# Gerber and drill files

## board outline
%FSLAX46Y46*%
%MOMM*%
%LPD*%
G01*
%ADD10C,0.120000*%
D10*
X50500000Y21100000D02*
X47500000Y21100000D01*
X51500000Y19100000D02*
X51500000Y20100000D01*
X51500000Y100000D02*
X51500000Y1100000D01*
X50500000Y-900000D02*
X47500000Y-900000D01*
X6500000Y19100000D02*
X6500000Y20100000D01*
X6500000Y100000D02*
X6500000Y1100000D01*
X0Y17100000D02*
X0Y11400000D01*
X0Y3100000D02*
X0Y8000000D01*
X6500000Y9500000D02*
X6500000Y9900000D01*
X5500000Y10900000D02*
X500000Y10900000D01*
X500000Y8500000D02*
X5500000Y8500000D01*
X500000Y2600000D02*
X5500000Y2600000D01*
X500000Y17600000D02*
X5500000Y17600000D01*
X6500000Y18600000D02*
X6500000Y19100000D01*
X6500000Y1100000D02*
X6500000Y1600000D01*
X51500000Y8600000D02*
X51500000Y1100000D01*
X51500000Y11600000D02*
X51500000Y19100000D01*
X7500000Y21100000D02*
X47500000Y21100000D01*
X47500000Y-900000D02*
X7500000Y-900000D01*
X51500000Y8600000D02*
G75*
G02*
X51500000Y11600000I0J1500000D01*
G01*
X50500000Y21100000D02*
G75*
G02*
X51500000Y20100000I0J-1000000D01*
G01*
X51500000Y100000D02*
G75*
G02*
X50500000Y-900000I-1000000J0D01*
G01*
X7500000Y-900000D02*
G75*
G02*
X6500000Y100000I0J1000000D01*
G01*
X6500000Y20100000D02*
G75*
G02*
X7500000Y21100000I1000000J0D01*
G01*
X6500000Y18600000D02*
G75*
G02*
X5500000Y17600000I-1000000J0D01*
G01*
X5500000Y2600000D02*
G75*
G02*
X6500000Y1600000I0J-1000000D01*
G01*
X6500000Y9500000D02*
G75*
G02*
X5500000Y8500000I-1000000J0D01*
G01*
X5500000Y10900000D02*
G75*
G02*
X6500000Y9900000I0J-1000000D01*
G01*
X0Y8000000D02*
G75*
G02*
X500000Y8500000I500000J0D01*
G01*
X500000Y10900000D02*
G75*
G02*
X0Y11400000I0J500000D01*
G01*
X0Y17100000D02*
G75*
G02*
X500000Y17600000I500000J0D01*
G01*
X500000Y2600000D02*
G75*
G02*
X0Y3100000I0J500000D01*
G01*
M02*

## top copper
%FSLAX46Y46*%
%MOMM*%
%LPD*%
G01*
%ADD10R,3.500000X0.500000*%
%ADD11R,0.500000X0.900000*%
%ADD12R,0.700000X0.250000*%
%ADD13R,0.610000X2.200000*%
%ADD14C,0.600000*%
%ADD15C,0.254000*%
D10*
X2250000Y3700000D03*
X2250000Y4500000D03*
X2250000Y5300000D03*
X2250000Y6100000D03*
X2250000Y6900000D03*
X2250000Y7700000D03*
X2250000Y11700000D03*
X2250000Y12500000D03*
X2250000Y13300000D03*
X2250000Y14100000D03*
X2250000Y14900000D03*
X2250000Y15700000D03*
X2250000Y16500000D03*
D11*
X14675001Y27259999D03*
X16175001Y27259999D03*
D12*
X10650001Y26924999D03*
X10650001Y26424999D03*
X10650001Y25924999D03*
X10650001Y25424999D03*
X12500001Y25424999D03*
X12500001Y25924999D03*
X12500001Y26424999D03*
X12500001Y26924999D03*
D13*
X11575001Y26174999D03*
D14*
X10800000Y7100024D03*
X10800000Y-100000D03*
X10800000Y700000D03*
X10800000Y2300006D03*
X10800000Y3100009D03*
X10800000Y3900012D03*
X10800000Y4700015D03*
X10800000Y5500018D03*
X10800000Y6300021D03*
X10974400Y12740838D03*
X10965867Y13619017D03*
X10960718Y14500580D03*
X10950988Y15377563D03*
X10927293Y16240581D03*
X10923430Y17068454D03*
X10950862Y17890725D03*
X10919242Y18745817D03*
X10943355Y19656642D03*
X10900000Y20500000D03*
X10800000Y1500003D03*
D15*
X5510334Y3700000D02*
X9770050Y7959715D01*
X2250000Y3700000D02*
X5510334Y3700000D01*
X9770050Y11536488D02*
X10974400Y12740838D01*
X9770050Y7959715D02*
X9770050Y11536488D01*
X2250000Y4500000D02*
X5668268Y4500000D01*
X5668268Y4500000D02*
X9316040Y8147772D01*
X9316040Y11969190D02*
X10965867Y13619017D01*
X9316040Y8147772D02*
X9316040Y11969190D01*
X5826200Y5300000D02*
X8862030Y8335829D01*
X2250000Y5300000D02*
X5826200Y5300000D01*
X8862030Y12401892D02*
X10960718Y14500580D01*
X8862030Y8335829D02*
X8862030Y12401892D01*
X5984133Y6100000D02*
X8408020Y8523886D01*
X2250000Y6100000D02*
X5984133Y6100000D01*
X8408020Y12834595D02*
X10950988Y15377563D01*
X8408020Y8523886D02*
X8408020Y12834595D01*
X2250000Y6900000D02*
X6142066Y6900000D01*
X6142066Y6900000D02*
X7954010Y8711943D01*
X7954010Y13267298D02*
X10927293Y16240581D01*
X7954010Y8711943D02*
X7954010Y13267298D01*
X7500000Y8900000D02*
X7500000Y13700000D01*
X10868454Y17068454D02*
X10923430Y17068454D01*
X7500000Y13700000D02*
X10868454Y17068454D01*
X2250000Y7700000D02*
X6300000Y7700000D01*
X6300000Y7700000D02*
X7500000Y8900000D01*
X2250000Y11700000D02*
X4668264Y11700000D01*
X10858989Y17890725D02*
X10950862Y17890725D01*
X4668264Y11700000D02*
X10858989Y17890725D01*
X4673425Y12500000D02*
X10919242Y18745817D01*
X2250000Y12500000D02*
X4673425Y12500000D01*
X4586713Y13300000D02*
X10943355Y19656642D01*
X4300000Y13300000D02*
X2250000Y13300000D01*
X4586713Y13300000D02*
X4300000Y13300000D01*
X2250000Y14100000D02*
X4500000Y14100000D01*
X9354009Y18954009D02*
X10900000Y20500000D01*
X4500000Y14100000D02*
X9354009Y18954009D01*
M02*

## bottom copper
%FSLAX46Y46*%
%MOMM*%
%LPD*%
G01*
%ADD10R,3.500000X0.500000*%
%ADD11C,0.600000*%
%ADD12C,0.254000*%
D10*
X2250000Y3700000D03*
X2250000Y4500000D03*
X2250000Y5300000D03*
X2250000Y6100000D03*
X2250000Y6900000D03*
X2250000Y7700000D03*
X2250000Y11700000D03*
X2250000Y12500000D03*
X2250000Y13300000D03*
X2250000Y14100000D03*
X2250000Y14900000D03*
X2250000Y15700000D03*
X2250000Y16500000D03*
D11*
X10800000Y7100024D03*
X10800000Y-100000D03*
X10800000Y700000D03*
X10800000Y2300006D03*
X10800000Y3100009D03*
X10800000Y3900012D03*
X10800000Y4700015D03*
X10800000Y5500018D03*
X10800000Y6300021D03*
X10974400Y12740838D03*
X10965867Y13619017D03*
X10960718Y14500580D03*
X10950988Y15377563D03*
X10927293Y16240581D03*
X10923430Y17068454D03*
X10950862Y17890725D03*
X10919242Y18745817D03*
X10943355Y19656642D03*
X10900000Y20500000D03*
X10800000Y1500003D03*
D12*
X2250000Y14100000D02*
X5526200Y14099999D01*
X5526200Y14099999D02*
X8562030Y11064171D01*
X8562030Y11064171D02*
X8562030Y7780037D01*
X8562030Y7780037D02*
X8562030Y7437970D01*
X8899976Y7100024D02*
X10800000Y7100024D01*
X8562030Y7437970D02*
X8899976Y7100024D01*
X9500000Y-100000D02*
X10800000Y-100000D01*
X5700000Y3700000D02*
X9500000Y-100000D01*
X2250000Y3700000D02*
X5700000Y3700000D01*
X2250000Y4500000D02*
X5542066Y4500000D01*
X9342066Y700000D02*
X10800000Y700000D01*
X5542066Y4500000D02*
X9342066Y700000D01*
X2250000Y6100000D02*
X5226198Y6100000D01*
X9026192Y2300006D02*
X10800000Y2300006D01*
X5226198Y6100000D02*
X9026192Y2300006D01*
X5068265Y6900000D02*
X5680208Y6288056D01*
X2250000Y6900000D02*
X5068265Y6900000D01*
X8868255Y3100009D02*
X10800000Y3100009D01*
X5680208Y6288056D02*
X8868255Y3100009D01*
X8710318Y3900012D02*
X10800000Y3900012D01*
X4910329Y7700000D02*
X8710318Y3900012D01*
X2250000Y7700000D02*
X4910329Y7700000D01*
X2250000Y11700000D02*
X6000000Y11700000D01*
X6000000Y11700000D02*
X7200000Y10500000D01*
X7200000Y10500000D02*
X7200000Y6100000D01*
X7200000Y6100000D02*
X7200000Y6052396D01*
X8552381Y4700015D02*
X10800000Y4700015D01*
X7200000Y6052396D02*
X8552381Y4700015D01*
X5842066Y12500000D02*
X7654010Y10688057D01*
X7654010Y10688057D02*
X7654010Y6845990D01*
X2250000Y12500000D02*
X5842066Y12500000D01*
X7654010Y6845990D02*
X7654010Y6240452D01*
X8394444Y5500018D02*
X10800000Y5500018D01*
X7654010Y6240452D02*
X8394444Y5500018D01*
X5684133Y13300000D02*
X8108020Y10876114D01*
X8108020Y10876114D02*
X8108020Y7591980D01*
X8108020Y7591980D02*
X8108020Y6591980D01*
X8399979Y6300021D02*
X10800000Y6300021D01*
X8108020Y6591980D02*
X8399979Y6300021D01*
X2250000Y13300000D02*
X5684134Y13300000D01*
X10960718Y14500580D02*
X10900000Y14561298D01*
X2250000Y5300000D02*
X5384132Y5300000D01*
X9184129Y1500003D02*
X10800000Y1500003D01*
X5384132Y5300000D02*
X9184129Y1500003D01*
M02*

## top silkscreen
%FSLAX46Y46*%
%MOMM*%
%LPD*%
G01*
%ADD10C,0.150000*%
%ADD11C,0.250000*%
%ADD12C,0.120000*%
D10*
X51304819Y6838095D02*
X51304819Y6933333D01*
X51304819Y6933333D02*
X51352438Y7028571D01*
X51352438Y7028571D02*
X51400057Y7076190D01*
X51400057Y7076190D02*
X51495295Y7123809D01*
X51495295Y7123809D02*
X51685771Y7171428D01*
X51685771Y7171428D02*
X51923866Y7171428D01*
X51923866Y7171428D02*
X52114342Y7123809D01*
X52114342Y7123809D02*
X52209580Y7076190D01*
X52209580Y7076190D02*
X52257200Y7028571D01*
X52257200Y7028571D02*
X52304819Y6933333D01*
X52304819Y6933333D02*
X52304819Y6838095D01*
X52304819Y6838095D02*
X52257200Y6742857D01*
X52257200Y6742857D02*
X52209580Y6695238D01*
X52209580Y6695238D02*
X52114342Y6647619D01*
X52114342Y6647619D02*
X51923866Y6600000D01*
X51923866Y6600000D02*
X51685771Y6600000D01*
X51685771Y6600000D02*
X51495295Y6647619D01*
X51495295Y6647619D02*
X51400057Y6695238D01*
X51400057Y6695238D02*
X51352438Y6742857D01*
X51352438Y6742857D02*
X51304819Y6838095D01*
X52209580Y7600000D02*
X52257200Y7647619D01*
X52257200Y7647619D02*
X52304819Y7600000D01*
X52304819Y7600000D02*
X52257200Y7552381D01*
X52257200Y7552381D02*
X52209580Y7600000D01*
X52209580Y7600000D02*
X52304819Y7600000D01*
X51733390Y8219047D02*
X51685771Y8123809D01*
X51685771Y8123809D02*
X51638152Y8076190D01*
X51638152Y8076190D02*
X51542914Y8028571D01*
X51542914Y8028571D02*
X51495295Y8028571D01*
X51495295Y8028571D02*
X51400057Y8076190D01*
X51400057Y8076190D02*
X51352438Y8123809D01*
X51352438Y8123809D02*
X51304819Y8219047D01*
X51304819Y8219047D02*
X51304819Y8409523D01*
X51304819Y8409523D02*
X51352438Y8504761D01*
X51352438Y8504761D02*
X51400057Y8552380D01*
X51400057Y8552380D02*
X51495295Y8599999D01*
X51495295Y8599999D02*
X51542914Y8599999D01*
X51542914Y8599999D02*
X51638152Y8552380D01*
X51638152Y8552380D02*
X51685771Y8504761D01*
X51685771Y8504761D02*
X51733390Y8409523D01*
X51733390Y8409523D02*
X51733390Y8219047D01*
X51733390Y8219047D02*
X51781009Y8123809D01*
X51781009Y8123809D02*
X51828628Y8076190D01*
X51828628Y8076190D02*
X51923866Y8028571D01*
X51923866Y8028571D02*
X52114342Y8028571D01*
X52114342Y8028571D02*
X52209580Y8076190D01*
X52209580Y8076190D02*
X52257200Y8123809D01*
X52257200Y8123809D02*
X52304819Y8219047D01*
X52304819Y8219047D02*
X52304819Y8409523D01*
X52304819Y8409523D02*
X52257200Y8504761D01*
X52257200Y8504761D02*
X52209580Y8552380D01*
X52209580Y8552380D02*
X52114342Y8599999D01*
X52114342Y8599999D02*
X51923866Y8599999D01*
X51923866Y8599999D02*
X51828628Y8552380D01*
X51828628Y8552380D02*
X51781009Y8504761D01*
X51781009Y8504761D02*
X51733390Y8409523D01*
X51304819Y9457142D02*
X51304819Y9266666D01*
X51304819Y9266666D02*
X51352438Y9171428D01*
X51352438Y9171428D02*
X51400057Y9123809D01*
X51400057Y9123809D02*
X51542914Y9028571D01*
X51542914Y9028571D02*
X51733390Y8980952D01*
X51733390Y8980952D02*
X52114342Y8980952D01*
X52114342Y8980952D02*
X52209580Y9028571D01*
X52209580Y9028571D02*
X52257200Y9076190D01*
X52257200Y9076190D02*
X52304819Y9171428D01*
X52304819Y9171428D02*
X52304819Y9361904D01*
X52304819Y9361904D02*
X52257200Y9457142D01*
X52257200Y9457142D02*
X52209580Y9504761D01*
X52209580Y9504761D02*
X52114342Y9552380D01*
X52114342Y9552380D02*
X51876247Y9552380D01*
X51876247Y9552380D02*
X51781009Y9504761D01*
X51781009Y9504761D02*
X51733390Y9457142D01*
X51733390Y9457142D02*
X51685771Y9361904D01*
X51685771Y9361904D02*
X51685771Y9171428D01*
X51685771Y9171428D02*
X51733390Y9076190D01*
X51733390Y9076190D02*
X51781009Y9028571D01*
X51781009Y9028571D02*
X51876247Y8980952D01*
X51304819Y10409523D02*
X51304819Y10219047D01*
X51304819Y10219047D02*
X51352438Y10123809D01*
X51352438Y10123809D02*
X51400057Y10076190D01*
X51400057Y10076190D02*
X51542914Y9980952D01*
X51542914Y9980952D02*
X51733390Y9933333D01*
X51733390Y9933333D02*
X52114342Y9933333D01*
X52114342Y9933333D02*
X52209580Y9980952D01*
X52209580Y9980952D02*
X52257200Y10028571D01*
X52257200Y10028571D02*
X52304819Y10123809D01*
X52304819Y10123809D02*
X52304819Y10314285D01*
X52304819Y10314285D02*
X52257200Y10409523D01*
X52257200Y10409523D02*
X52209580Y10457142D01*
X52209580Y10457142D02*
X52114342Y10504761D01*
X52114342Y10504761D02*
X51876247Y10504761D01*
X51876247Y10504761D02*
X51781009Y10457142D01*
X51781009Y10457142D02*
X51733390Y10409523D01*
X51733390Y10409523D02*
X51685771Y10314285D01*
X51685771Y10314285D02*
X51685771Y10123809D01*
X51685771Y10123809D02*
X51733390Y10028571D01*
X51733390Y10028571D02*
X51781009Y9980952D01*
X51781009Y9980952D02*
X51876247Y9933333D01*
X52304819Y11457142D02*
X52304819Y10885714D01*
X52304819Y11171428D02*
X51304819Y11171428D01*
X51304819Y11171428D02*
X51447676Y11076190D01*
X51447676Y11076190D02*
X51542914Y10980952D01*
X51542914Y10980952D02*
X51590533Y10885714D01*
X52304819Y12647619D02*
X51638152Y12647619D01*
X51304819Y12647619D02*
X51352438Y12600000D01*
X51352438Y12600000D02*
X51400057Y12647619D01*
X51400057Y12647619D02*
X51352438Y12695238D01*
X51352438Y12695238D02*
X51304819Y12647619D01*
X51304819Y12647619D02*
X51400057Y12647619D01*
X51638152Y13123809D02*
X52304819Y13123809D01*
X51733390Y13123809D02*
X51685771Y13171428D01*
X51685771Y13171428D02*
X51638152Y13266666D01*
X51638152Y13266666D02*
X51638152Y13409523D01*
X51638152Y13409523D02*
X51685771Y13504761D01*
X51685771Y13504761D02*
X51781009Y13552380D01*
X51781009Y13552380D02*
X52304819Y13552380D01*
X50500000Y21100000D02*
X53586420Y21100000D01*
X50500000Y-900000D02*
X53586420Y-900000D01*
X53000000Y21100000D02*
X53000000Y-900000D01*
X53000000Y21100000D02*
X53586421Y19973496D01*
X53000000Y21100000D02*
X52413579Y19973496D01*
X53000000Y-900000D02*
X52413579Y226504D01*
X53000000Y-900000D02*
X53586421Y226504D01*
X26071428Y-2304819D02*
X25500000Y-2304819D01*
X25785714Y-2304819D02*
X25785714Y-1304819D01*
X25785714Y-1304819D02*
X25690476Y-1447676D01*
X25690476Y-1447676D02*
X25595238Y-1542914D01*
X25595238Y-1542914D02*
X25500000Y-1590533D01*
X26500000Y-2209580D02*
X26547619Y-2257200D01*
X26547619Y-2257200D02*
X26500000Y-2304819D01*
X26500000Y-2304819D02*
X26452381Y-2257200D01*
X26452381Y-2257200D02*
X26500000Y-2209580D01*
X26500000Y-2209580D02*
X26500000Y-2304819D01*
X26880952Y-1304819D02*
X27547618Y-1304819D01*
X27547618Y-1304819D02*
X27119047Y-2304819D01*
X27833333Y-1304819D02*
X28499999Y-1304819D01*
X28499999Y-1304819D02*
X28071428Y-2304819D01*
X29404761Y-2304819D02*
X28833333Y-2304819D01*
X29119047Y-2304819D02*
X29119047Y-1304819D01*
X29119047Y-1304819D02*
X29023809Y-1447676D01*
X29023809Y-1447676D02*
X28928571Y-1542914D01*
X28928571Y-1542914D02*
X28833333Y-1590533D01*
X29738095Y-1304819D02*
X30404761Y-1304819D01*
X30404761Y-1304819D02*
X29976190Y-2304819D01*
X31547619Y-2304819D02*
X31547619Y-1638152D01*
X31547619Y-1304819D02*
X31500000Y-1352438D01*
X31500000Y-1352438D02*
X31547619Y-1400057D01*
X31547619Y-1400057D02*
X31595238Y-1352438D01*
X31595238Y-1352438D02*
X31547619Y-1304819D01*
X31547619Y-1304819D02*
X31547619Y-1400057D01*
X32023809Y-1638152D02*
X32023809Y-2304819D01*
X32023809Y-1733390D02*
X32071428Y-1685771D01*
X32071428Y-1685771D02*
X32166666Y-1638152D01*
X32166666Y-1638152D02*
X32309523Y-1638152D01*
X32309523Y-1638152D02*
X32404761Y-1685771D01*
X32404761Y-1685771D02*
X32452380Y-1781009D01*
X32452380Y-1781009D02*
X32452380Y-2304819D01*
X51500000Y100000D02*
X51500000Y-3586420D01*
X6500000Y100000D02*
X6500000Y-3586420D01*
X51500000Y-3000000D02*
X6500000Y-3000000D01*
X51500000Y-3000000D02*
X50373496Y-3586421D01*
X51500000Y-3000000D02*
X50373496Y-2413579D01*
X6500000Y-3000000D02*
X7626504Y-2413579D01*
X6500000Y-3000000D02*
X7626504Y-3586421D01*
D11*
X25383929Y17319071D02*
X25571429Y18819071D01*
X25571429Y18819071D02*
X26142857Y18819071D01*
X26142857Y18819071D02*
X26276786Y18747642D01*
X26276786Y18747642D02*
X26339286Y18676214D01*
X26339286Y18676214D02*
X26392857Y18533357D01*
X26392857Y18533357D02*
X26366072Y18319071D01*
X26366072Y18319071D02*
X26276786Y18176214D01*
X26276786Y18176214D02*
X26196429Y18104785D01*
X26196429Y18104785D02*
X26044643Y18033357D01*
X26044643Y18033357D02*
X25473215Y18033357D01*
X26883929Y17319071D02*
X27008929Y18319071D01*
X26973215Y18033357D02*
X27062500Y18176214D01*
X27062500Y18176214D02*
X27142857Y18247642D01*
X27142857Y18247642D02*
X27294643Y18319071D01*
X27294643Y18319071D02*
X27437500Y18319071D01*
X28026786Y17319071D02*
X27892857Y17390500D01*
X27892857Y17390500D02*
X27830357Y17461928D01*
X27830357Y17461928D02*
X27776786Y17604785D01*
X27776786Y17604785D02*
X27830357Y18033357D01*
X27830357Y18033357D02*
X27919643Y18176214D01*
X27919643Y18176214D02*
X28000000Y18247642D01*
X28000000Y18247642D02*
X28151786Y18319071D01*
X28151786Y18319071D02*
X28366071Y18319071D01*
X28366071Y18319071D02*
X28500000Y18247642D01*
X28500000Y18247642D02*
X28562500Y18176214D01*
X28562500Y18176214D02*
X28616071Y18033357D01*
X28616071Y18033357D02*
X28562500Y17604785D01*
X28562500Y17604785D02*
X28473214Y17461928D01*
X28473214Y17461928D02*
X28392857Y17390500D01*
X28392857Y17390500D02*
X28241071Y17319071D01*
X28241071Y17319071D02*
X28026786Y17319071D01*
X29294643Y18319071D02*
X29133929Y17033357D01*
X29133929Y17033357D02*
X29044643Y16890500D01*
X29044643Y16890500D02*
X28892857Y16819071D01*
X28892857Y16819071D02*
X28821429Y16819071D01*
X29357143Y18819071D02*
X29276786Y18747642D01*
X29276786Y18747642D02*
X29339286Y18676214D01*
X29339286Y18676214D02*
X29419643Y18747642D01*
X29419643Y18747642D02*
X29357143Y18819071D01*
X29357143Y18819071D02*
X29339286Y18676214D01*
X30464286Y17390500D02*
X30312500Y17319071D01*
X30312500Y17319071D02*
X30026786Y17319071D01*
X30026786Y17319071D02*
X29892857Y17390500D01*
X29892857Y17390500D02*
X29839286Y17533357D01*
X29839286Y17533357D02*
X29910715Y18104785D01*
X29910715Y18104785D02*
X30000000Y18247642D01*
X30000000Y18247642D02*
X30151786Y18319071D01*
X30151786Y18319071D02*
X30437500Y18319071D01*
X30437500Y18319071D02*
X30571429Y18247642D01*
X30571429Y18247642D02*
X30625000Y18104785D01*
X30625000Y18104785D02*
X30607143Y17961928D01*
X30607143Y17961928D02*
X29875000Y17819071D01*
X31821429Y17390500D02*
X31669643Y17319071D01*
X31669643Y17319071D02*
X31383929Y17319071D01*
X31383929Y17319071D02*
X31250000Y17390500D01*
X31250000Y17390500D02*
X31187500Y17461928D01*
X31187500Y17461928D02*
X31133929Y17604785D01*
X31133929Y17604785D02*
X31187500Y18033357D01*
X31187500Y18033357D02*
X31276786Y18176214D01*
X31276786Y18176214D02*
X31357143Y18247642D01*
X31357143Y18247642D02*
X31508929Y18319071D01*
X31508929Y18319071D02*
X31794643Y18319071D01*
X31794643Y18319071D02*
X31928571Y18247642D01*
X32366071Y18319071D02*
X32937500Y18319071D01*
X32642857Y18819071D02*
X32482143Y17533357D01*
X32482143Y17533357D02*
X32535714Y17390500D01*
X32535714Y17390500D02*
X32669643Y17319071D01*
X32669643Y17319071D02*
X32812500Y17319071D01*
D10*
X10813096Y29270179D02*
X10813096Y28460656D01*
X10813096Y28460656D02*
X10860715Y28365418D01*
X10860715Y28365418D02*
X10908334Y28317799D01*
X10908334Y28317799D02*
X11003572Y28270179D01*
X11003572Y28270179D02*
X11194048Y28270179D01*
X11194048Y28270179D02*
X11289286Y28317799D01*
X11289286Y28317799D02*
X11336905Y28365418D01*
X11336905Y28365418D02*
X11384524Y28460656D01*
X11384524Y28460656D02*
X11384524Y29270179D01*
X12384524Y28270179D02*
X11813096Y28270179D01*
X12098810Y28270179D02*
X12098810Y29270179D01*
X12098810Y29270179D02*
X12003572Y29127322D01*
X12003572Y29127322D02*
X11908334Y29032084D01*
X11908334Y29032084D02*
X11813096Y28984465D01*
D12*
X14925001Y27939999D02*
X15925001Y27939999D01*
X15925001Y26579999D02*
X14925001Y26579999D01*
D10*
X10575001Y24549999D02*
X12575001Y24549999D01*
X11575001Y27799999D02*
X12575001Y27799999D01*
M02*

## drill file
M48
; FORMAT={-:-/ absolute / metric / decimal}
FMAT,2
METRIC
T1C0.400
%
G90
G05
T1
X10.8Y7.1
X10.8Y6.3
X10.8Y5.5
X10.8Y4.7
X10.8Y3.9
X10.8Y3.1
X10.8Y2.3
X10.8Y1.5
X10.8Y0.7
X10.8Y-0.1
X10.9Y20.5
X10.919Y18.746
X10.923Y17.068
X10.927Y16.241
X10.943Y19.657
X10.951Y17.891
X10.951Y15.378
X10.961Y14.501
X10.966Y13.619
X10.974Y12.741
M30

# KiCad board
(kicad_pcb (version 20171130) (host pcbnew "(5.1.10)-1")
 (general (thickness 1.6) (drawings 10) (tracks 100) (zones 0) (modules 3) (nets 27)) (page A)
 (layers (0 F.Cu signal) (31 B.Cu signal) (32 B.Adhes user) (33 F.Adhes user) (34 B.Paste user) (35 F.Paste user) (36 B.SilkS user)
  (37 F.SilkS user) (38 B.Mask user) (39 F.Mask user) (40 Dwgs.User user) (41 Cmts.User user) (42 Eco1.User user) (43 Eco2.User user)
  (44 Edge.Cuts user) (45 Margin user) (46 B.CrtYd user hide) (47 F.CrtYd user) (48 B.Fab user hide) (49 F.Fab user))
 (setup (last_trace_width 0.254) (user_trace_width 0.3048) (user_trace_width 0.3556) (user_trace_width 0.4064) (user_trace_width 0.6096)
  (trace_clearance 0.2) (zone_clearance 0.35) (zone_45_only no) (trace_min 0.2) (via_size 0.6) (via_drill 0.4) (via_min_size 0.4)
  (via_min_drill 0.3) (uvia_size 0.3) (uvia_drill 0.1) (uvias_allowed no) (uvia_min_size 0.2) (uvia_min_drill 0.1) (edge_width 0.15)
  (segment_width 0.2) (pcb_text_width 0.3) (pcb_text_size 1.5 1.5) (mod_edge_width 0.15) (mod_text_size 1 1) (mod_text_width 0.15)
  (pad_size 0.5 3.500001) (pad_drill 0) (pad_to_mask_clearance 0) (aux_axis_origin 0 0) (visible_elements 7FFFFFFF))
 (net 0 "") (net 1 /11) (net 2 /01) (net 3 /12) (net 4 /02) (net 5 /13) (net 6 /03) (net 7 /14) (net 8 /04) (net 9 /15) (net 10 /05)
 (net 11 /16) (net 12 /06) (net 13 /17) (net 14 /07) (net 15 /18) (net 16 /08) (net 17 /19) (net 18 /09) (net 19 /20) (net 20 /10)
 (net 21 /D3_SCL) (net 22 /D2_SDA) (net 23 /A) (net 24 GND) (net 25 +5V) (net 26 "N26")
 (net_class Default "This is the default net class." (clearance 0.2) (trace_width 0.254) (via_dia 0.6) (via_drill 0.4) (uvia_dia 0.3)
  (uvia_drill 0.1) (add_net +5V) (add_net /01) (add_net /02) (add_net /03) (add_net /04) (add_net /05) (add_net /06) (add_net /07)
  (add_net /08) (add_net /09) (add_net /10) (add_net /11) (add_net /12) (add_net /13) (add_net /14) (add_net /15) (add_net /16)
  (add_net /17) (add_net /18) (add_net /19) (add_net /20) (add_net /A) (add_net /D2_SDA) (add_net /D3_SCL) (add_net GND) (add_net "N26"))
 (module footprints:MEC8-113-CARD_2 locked (layer F.Cu) (at 0 -0.1 90)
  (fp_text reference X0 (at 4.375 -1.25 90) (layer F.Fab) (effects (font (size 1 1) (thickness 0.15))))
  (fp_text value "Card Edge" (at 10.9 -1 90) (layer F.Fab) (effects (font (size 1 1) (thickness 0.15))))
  (fp_line (start 21 50.5) (end 21 47.5) (layer Edge.Cuts) (width 0.12))
  (fp_line (start 19 51.5) (end 20 51.5) (layer Edge.Cuts) (width 0.12))
  (fp_line (start 0 51.5) (end 1 51.5) (layer Edge.Cuts) (width 0.12))
  (fp_line (start -1 50.5) (end -1 47.5) (layer Edge.Cuts) (width 0.12))
  (fp_line (start 19 6.5) (end 20 6.5) (layer Edge.Cuts) (width 0.12))
  (fp_line (start 0 6.5) (end 1 6.5) (layer Edge.Cuts) (width 0.12))
  (fp_line (start 17 0) (end 11.3 0) (layer Edge.Cuts) (width 0.12))
  (fp_line (start 3 0) (end 7.9 0) (layer Edge.Cuts) (width 0.12))
  (fp_line (start 9.4 6.5) (end 9.8 6.5) (layer Edge.Cuts) (width 0.12))
  (fp_line (start 10.8 5.5) (end 10.8 0.5) (layer Edge.Cuts) (width 0.12))
  (fp_line (start 8.4 0.5) (end 8.4 5.5) (layer Edge.Cuts) (width 0.12))
  (fp_line (start 2.5 0.5) (end 2.5 5.5) (layer Edge.Cuts) (width 0.12))
  (fp_line (start 17.5 0.5) (end 17.5 5.5) (layer Edge.Cuts) (width 0.12))
  (fp_line (start 18.5 6.5) (end 19 6.5) (layer Edge.Cuts) (width 0.12))
  (fp_line (start 1 6.5) (end 1.5 6.5) (layer Edge.Cuts) (width 0.12))
  (fp_line (start 8.5 51.5) (end 1 51.5) (layer Edge.Cuts) (width 0.12))
  (fp_line (start 11.5 51.5) (end 19 51.5) (layer Edge.Cuts) (width 0.12))
  (fp_line (start 21 7.5) (end 21 47.5) (layer Edge.Cuts) (width 0.12))
  (fp_line (start -1 47.5) (end -1 7.5) (layer Edge.Cuts) (width 0.12))
  (fp_arc (start 10 51.5) (end 11.5 51.5) (angle -180) (layer Edge.Cuts) (width 0.12))
  (fp_arc (start 20 50.5) (end 20 51.5) (angle -90) (layer Edge.Cuts) (width 0.12))
  (fp_arc (start 0 50.5) (end -1 50.5) (angle -90) (layer Edge.Cuts) (width 0.12))
  (fp_arc (start 0 7.5) (end 0 6.5) (angle -90) (layer Edge.Cuts) (width 0.12))
  (fp_arc (start 20 7.5) (end 21 7.5) (angle -90) (layer Edge.Cuts) (width 0.12))
  (fp_arc (start 18.5 5.5) (end 17.5 5.5) (angle -90) (layer Edge.Cuts) (width 0.12))
  (fp_arc (start 1.5 5.5) (end 1.5 6.5) (angle -90) (layer Edge.Cuts) (width 0.12))
  (fp_arc (start 9.4 5.5) (end 8.4 5.5) (angle -90) (layer Edge.Cuts) (width 0.12))
  (fp_arc (start 9.8 5.5) (end 9.8 6.5) (angle -90) (layer Edge.Cuts) (width 0.12))
  (fp_arc (start 7.9 0.5) (end 8.4 0.5) (angle -90) (layer Edge.Cuts) (width 0.12))
  (fp_arc (start 11.3 0.5) (end 11.3 0) (angle -90) (layer Edge.Cuts) (width 0.12))
  (fp_arc (start 17 0.5) (end 17.5 0.5) (angle -90) (layer Edge.Cuts) (width 0.12))
  (fp_arc (start 3 0.5) (end 3 0) (angle -90) (layer Edge.Cuts) (width 0.12))
  (pad 14 smd rect (at 3.6 2.25 90) (size 0.5 3.5) (layers F.Cu F.Paste F.Mask) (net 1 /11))
  (pad 1 smd rect (at 3.6 2.25 90) (size 0.5 3.5) (layers B.Cu B.Paste B.Mask) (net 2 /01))
  (pad 15 smd rect (at 4.4 2.25 90) (size 0.5 3.5) (layers F.Cu F.Paste F.Mask) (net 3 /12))
  (pad 2 smd rect (at 4.4 2.25 90) (size 0.5 3.5) (layers B.Cu B.Paste B.Mask) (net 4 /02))
  (pad 16 smd rect (at 5.2 2.25 90) (size 0.5 3.5) (layers F.Cu F.Paste F.Mask) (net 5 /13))
  (pad 3 smd rect (at 5.2 2.25 90) (size 0.5 3.5) (layers B.Cu B.Paste B.Mask) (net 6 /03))
  (pad 17 smd rect (at 6 2.25 90) (size 0.5 3.5) (layers F.Cu F.Paste F.Mask) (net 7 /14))
  (pad 4 smd rect (at 6 2.25 90) (size 0.5 3.5) (layers B.Cu B.Paste B.Mask) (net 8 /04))
  (pad 18 smd rect (at 6.8 2.25 90) (size 0.5 3.5) (layers F.Cu F.Paste F.Mask) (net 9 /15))
  (pad 5 smd rect (at 6.8 2.25 90) (size 0.5 3.5) (layers B.Cu B.Paste B.Mask) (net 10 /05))
  (pad 19 smd rect (at 7.6 2.25 90) (size 0.5 3.5) (layers F.Cu F.Paste F.Mask) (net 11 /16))
  (pad 6 smd rect (at 7.6 2.25 90) (size 0.5 3.5) (layers B.Cu B.Paste B.Mask) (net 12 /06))
  (pad 20 smd rect (at 11.6 2.25 90) (size 0.5 3.5) (layers F.Cu F.Paste F.Mask) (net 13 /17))
  (pad 7 smd rect (at 11.6 2.25 90) (size 0.5 3.5) (layers B.Cu B.Paste B.Mask) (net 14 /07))
  (pad 21 smd rect (at 12.4 2.25 90) (size 0.5 3.5) (layers F.Cu F.Paste F.Mask) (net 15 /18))
  (pad 8 smd rect (at 12.4 2.25 90) (size 0.5 3.5) (layers B.Cu B.Paste B.Mask) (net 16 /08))
  (pad 22 smd rect (at 13.2 2.25 90) (size 0.5 3.5) (layers F.Cu F.Paste F.Mask) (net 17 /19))
  (pad 9 smd rect (at 13.2 2.25 90) (size 0.5 3.5) (layers B.Cu B.Paste B.Mask) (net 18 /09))
  (pad 23 smd rect (at 14 2.25 90) (size 0.5 3.5) (layers F.Cu F.Paste F.Mask) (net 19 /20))
  (pad 10 smd rect (at 14 2.25 90) (size 0.5 3.5) (layers B.Cu B.Paste B.Mask) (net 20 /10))
  (pad 24 smd rect (at 14.8 2.25 90) (size 0.5 3.5) (layers F.Cu F.Paste F.Mask) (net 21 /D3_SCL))
  (pad 11 smd rect (at 14.8 2.25 90) (size 0.5 3.5) (layers B.Cu B.Paste B.Mask))
  (pad 25 smd rect (at 15.6 2.25 90) (size 0.5 3.5) (layers F.Cu F.Paste F.Mask) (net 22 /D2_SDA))
  (pad 12 smd rect (at 15.6 2.25 90) (size 0.5 3.5) (layers B.Cu B.Paste B.Mask) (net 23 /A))
  (pad 26 smd rect (at 16.4 2.25 90) (size 0.5 3.5) (layers F.Cu F.Paste F.Mask) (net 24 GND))
  (pad 13 smd rect (at 16.4 2.25 90) (size 0.5 3.5) (layers B.Cu B.Paste B.Mask) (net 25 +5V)))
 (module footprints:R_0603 (layer F.Cu) (at 15.425001 -27.259999)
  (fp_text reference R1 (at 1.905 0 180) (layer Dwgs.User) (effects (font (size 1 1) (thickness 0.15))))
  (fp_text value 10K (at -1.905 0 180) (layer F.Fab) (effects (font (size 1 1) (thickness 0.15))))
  (fp_line (start -0.5 -0.68) (end 0.5 -0.68) (layer F.SilkS) (width 0.12))
  (fp_line (start 0.5 0.68) (end -0.5 0.68) (layer F.SilkS) (width 0.12))
  (pad 1 smd rect (at -0.75 0) (size 0.5 0.9) (layers F.Cu F.Paste F.Mask) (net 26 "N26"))
  (pad 2 smd rect (at 0.75 0) (size 0.5 0.9) (layers F.Cu F.Paste F.Mask) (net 23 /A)))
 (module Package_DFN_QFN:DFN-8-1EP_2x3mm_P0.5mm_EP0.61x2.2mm (layer F.Cu) (at 11.575001 -26.174999)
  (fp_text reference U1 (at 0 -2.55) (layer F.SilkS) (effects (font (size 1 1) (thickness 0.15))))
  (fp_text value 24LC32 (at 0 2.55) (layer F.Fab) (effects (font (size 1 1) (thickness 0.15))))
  (fp_line (start -1 1.625) (end 1 1.625) (layer F.SilkS) (width 0.15))
  (fp_line (start 0 -1.625) (end 1 -1.625) (layer F.SilkS) (width 0.15))
  (pad 1 smd rect (at -0.925 -0.75) (size 0.7 0.25) (layers F.Cu F.Paste F.Mask) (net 26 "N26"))
  (pad 2 smd rect (at -0.925 -0.25) (size 0.7 0.25) (layers F.Cu F.Paste F.Mask) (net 24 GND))
  (pad 3 smd rect (at -0.925 0.25) (size 0.7 0.25) (layers F.Cu F.Paste F.Mask) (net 24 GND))
  (pad 4 smd rect (at -0.925 0.75) (size 0.7 0.25) (layers F.Cu F.Paste F.Mask) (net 24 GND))
  (pad 5 smd rect (at 0.925 0.75) (size 0.7 0.25) (layers F.Cu F.Paste F.Mask) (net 22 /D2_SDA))
  (pad 6 smd rect (at 0.925 0.25) (size 0.7 0.25) (layers F.Cu F.Paste F.Mask) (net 21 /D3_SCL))
  (pad 7 smd rect (at 0.925 -0.25) (size 0.7 0.25) (layers F.Cu F.Paste F.Mask))
  (pad 8 smd rect (at 0.925 -0.75) (size 0.7 0.25) (layers F.Cu F.Paste F.Mask) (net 25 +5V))
  (pad 9 smd rect (at 0 0) (size 0.61 2.2) (layers F.Cu F.Mask))
  (pad "" smd rect (at 0 -0.734) (size 0.5 0.59) (layers F.Paste)) (pad "" smd rect (at 0 0) (size 0.5 0.59) (layers F.Paste))
  (pad "" smd rect (at 0 0.734) (size 0.5 0.59) (layers F.Paste)))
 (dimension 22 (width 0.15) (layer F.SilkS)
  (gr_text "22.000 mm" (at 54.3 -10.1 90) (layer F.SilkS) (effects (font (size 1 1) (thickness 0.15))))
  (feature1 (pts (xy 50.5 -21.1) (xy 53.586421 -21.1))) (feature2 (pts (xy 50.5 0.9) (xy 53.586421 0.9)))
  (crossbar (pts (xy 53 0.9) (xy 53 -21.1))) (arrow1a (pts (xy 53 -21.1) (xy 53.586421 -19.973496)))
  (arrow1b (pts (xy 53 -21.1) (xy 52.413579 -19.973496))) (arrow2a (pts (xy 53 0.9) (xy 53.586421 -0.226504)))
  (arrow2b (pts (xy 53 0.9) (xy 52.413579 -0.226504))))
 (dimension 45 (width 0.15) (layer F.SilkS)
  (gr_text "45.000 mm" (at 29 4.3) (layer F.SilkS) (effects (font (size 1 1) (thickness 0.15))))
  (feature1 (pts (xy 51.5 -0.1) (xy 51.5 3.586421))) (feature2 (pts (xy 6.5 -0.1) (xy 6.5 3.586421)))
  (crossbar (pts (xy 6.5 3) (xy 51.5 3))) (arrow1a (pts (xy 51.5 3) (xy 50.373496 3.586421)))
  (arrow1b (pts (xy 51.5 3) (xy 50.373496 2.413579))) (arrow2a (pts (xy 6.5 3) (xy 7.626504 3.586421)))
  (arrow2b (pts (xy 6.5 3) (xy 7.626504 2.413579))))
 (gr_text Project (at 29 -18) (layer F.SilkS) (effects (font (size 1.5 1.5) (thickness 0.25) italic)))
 (segment (start 2.25 -14.1) (end 5.5262 -14.099999) (width 0.254) (layer B.Cu) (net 20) (status 10))
 (segment (start 5.5262 -14.099999) (end 8.56203 -11.064171) (width 0.254) (layer B.Cu) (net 20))
 (segment (start 8.56203 -11.064171) (end 8.56203 -7.780037) (width 0.254) (layer B.Cu) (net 20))
 (segment (start 8.56203 -7.780037) (end 8.56203 -7.43797) (width 0.254) (layer B.Cu) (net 20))
 (via (at 10.8 -7.100024) (size 0.6) (drill 0.4) (layers F.Cu B.Cu) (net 20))
 (segment (start 8.899976 -7.100024) (end 10.8 -7.100024) (width 0.254) (layer B.Cu) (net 20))
 (segment (start 8.56203 -7.43797) (end 8.899976 -7.100024) (width 0.254) (layer B.Cu) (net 20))
 (via (at 10.8 0.1) (size 0.6) (drill 0.4) (layers F.Cu B.Cu) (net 2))
 (segment (start 9.5 0.1) (end 10.8 0.1) (width 0.254) (layer B.Cu) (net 2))
 (segment (start 5.7 -3.7) (end 9.5 0.1) (width 0.254) (layer B.Cu) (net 2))
 (segment (start 2.25 -3.7) (end 5.7 -3.7) (width 0.254) (layer B.Cu) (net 2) (status 10))
 (segment (start 2.25 -4.5) (end 5.542066 -4.5) (width 0.254) (layer B.Cu) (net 4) (status 10))
 (via (at 10.8 -0.7) (size 0.6) (drill 0.4) (layers F.Cu B.Cu) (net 4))
 (segment (start 9.342066 -0.7) (end 10.8 -0.7) (width 0.254) (layer B.Cu) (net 4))
 (segment (start 5.542066 -4.5) (end 9.342066 -0.7) (width 0.254) (layer B.Cu) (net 4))
 (segment (start 2.25 -6.1) (end 5.226198 -6.1) (width 0.254) (layer B.Cu) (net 8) (status 10))
 (via (at 10.8 -2.300006) (size 0.6) (drill 0.4) (layers F.Cu B.Cu) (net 8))
 (segment (start 9.026192 -2.300006) (end 10.8 -2.300006) (width 0.254) (layer B.Cu) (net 8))
 (segment (start 5.226198 -6.1) (end 9.026192 -2.300006) (width 0.254) (layer B.Cu) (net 8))
 (segment (start 5.068265 -6.9) (end 5.680208 -6.288056) (width 0.254) (layer B.Cu) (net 10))
 (segment (start 2.25 -6.9) (end 5.068265 -6.9) (width 0.254) (layer B.Cu) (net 10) (status 10))
 (via (at 10.8 -3.100009) (size 0.6) (drill 0.4) (layers F.Cu B.Cu) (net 10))
 (segment (start 8.868255 -3.100009) (end 10.8 -3.100009) (width 0.254) (layer B.Cu) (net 10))
 (segment (start 5.680208 -6.288056) (end 8.868255 -3.100009) (width 0.254) (layer B.Cu) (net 10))
 (via (at 10.8 -3.900012) (size 0.6) (drill 0.4) (layers F.Cu B.Cu) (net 12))
 (segment (start 8.710318 -3.900012) (end 10.8 -3.900012) (width 0.254) (layer B.Cu) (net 12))
 (segment (start 4.910329 -7.7) (end 8.710318 -3.900012) (width 0.254) (layer B.Cu) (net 12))
 (segment (start 2.25 -7.7) (end 4.910329 -7.7) (width 0.254) (layer B.Cu) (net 12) (status 10))
 (segment (start 2.25 -11.7) (end 6 -11.7) (width 0.254) (layer B.Cu) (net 14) (status 10))
 (segment (start 6 -11.7) (end 7.2 -10.5) (width 0.254) (layer B.Cu) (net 14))
 (segment (start 7.2 -10.5) (end 7.2 -6.1) (width 0.254) (layer B.Cu) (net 14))
 (segment (start 7.2 -6.1) (end 7.2 -6.052396) (width 0.254) (layer B.Cu) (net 14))
 (via (at 10.8 -4.700015) (size 0.6) (drill 0.4) (layers F.Cu B.Cu) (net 14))
 (segment (start 8.552381 -4.700015) (end 10.8 -4.700015) (width 0.254) (layer B.Cu) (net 14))
 (segment (start 7.2 -6.052396) (end 8.552381 -4.700015) (width 0.254) (layer B.Cu) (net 14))
 (segment (start 5.842066 -12.5) (end 7.65401 -10.688057) (width 0.254) (layer B.Cu) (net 16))
 (segment (start 7.65401 -10.688057) (end 7.65401 -6.84599) (width 0.254) (layer B.Cu) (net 16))
 (segment (start 2.25 -12.5) (end 5.842066 -12.5) (width 0.254) (layer B.Cu) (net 16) (status 10))
 (segment (start 7.65401 -6.84599) (end 7.65401 -6.240452) (width 0.254) (layer B.Cu) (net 16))
 (segment (start 8.394444 -5.500018) (end 10.8 -5.500018) (width 0.254) (layer B.Cu) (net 16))
 (via (at 10.8 -5.500018) (size 0.6) (drill 0.4) (layers F.Cu B.Cu) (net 16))
 (segment (start 7.65401 -6.240452) (end 8.394444 -5.500018) (width 0.254) (layer B.Cu) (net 16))
 (segment (start 5.684133 -13.3) (end 8.10802 -10.876114) (width 0.254) (layer B.Cu) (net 18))
 (segment (start 8.10802 -10.876114) (end 8.10802 -7.59198) (width 0.254) (layer B.Cu) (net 18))
 (segment (start 8.10802 -7.59198) (end 8.10802 -6.59198) (width 0.254) (layer B.Cu) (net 18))
 (via (at 10.8 -6.300021) (size 0.6) (drill 0.4) (layers F.Cu B.Cu) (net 18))
 (segment (start 8.399979 -6.300021) (end 10.8 -6.300021) (width 0.254) (layer B.Cu) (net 18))
 (segment (start 8.10802 -6.59198) (end 8.399979 -6.300021) (width 0.254) (layer B.Cu) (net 18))
 (segment (start 2.25 -13.3) (end 5.684134 -13.3) (width 0.254) (layer B.Cu) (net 18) (status 10))
 (segment (start 5.510334 -3.7) (end 9.77005 -7.959715) (width 0.254) (layer F.Cu) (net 1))
 (segment (start 2.25 -3.7) (end 5.510334 -3.7) (width 0.254) (layer F.Cu) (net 1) (status 10))
 (via (at 10.9744 -12.740838) (size 0.6) (drill 0.4) (layers F.Cu B.Cu) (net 1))
 (segment (start 9.77005 -11.536488) (end 10.9744 -12.740838) (width 0.254) (layer F.Cu) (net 1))
 (segment (start 9.77005 -7.959715) (end 9.77005 -11.536488) (width 0.254) (layer F.Cu) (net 1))
 (segment (start 2.25 -4.5) (end 5.668268 -4.5) (width 0.254) (layer F.Cu) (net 3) (status 10))
 (segment (start 5.668268 -4.5) (end 9.31604 -8.147772) (width 0.254) (layer F.Cu) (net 3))
 (via (at 10.965867 -13.619017) (size 0.6) (drill 0.4) (layers F.Cu B.Cu) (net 3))
 (segment (start 9.31604 -11.96919) (end 10.965867 -13.619017) (width 0.254) (layer F.Cu) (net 3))
 (segment (start 9.31604 -8.147772) (end 9.31604 -11.96919) (width 0.254) (layer F.Cu) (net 3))
 (segment (start 5.8262 -5.3) (end 8.86203 -8.335829) (width 0.254) (layer F.Cu) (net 5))
 (segment (start 2.25 -5.3) (end 5.8262 -5.3) (width 0.254) (layer F.Cu) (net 5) (status 10))
 (via (at 10.960718 -14.50058) (size 0.6) (drill 0.4) (layers F.Cu B.Cu) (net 5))
 (segment (start 8.86203 -12.401892) (end 10.960718 -14.50058) (width 0.254) (layer F.Cu) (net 5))
 (segment (start 8.86203 -8.335829) (end 8.86203 -12.401892) (width 0.254) (layer F.Cu) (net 5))
 (segment (start 10.960718 -14.50058) (end 10.9 -14.561298) (width 0.254) (layer B.Cu) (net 5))
 (segment (start 5.984133 -6.1) (end 8.40802 -8.523886) (width 0.254) (layer F.Cu) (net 7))
 (segment (start 2.25 -6.1) (end 5.984133 -6.1) (width 0.254) (layer F.Cu) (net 7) (status 10))
 (via (at 10.950988 -15.377563) (size 0.6) (drill 0.4) (layers F.Cu B.Cu) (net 7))
 (segment (start 8.40802 -12.834595) (end 10.950988 -15.377563) (width 0.254) (layer F.Cu) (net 7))
 (segment (start 8.40802 -8.523886) (end 8.40802 -12.834595) (width 0.254) (layer F.Cu) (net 7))
 (segment (start 2.25 -6.9) (end 6.142066 -6.9) (width 0.254) (layer F.Cu) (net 9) (status 10))
 (segment (start 6.142066 -6.9) (end 7.95401 -8.711943) (width 0.254) (layer F.Cu) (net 9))
 (via (at 10.927293 -16.240581) (size 0.6) (drill 0.4) (layers F.Cu B.Cu) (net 9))
 (segment (start 7.95401 -13.267298) (end 10.927293 -16.240581) (width 0.254) (layer F.Cu) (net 9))
 (segment (start 7.95401 -8.711943) (end 7.95401 -13.267298) (width 0.254) (layer F.Cu) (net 9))
 (segment (start 7.5 -8.9) (end 7.5 -13.7) (width 0.254) (layer F.Cu) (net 11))
 (via (at 10.92343 -17.068454) (size 0.6) (drill 0.4) (layers F.Cu B.Cu) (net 11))
 (segment (start 10.868454 -17.068454) (end 10.92343 -17.068454) (width 0.254) (layer F.Cu) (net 11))
 (segment (start 7.5 -13.7) (end 10.868454 -17.068454) (width 0.254) (layer F.Cu) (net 11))
 (segment (start 2.25 -7.7) (end 6.3 -7.7) (width 0.254) (layer F.Cu) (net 11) (status 10))
 (segment (start 6.3 -7.7) (end 7.5 -8.9) (width 0.254) (layer F.Cu) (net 11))
 (via (at 10.950862 -17.890725) (size 0.6) (drill 0.4) (layers F.Cu B.Cu) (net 13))
 (segment (start 2.25 -11.7) (end 4.668264 -11.7) (width 0.254) (layer F.Cu) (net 13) (status 10))
 (segment (start 10.858989 -17.890725) (end 10.950862 -17.890725) (width 0.254) (layer F.Cu) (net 13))
 (segment (start 4.668264 -11.7) (end 10.858989 -17.890725) (width 0.254) (layer F.Cu) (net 13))
 (via (at 10.919242 -18.745817) (size 0.6) (drill 0.4) (layers F.Cu B.Cu) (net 15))
 (segment (start 4.673425 -12.5) (end 10.919242 -18.745817) (width 0.254) (layer F.Cu) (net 15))
 (segment (start 2.25 -12.5) (end 4.673425 -12.5) (width 0.254) (layer F.Cu) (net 15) (status 10))
 (via (at 10.943355 -19.656642) (size 0.6) (drill 0.4) (layers F.Cu B.Cu) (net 17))
 (segment (start 4.586713 -13.3) (end 10.943355 -19.656642) (width 0.254) (layer F.Cu) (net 17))
 (segment (start 4.3 -13.3) (end 2.25 -13.3) (width 0.254) (layer F.Cu) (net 17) (status 20))
 (segment (start 4.586713 -13.3) (end 4.3 -13.3) (width 0.254) (layer F.Cu) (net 17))
 (segment (start 2.25 -14.1) (end 4.5 -14.1) (width 0.254) (layer F.Cu) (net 19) (status 10))
 (via (at 10.9 -20.5) (size 0.6) (drill 0.4) (layers F.Cu B.Cu) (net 19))
 (segment (start 9.354009 -18.954009) (end 10.9 -20.5) (width 0.254) (layer F.Cu) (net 19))
 (segment (start 4.5 -14.1) (end 9.354009 -18.954009) (width 0.254) (layer F.Cu) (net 19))
 (segment (start 2.25 -5.3) (end 5.384132 -5.3) (width 0.254) (layer B.Cu) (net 6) (status 10))
 (via (at 10.8 -1.500003) (size 0.6) (drill 0.4) (layers F.Cu B.Cu) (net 6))
 (segment (start 9.184129 -1.500003) (end 10.8 -1.500003) (width 0.254) (layer B.Cu) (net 6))
 (segment (start 5.384132 -5.3) (end 9.184129 -1.500003) (width 0.254) (layer B.Cu) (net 6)))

